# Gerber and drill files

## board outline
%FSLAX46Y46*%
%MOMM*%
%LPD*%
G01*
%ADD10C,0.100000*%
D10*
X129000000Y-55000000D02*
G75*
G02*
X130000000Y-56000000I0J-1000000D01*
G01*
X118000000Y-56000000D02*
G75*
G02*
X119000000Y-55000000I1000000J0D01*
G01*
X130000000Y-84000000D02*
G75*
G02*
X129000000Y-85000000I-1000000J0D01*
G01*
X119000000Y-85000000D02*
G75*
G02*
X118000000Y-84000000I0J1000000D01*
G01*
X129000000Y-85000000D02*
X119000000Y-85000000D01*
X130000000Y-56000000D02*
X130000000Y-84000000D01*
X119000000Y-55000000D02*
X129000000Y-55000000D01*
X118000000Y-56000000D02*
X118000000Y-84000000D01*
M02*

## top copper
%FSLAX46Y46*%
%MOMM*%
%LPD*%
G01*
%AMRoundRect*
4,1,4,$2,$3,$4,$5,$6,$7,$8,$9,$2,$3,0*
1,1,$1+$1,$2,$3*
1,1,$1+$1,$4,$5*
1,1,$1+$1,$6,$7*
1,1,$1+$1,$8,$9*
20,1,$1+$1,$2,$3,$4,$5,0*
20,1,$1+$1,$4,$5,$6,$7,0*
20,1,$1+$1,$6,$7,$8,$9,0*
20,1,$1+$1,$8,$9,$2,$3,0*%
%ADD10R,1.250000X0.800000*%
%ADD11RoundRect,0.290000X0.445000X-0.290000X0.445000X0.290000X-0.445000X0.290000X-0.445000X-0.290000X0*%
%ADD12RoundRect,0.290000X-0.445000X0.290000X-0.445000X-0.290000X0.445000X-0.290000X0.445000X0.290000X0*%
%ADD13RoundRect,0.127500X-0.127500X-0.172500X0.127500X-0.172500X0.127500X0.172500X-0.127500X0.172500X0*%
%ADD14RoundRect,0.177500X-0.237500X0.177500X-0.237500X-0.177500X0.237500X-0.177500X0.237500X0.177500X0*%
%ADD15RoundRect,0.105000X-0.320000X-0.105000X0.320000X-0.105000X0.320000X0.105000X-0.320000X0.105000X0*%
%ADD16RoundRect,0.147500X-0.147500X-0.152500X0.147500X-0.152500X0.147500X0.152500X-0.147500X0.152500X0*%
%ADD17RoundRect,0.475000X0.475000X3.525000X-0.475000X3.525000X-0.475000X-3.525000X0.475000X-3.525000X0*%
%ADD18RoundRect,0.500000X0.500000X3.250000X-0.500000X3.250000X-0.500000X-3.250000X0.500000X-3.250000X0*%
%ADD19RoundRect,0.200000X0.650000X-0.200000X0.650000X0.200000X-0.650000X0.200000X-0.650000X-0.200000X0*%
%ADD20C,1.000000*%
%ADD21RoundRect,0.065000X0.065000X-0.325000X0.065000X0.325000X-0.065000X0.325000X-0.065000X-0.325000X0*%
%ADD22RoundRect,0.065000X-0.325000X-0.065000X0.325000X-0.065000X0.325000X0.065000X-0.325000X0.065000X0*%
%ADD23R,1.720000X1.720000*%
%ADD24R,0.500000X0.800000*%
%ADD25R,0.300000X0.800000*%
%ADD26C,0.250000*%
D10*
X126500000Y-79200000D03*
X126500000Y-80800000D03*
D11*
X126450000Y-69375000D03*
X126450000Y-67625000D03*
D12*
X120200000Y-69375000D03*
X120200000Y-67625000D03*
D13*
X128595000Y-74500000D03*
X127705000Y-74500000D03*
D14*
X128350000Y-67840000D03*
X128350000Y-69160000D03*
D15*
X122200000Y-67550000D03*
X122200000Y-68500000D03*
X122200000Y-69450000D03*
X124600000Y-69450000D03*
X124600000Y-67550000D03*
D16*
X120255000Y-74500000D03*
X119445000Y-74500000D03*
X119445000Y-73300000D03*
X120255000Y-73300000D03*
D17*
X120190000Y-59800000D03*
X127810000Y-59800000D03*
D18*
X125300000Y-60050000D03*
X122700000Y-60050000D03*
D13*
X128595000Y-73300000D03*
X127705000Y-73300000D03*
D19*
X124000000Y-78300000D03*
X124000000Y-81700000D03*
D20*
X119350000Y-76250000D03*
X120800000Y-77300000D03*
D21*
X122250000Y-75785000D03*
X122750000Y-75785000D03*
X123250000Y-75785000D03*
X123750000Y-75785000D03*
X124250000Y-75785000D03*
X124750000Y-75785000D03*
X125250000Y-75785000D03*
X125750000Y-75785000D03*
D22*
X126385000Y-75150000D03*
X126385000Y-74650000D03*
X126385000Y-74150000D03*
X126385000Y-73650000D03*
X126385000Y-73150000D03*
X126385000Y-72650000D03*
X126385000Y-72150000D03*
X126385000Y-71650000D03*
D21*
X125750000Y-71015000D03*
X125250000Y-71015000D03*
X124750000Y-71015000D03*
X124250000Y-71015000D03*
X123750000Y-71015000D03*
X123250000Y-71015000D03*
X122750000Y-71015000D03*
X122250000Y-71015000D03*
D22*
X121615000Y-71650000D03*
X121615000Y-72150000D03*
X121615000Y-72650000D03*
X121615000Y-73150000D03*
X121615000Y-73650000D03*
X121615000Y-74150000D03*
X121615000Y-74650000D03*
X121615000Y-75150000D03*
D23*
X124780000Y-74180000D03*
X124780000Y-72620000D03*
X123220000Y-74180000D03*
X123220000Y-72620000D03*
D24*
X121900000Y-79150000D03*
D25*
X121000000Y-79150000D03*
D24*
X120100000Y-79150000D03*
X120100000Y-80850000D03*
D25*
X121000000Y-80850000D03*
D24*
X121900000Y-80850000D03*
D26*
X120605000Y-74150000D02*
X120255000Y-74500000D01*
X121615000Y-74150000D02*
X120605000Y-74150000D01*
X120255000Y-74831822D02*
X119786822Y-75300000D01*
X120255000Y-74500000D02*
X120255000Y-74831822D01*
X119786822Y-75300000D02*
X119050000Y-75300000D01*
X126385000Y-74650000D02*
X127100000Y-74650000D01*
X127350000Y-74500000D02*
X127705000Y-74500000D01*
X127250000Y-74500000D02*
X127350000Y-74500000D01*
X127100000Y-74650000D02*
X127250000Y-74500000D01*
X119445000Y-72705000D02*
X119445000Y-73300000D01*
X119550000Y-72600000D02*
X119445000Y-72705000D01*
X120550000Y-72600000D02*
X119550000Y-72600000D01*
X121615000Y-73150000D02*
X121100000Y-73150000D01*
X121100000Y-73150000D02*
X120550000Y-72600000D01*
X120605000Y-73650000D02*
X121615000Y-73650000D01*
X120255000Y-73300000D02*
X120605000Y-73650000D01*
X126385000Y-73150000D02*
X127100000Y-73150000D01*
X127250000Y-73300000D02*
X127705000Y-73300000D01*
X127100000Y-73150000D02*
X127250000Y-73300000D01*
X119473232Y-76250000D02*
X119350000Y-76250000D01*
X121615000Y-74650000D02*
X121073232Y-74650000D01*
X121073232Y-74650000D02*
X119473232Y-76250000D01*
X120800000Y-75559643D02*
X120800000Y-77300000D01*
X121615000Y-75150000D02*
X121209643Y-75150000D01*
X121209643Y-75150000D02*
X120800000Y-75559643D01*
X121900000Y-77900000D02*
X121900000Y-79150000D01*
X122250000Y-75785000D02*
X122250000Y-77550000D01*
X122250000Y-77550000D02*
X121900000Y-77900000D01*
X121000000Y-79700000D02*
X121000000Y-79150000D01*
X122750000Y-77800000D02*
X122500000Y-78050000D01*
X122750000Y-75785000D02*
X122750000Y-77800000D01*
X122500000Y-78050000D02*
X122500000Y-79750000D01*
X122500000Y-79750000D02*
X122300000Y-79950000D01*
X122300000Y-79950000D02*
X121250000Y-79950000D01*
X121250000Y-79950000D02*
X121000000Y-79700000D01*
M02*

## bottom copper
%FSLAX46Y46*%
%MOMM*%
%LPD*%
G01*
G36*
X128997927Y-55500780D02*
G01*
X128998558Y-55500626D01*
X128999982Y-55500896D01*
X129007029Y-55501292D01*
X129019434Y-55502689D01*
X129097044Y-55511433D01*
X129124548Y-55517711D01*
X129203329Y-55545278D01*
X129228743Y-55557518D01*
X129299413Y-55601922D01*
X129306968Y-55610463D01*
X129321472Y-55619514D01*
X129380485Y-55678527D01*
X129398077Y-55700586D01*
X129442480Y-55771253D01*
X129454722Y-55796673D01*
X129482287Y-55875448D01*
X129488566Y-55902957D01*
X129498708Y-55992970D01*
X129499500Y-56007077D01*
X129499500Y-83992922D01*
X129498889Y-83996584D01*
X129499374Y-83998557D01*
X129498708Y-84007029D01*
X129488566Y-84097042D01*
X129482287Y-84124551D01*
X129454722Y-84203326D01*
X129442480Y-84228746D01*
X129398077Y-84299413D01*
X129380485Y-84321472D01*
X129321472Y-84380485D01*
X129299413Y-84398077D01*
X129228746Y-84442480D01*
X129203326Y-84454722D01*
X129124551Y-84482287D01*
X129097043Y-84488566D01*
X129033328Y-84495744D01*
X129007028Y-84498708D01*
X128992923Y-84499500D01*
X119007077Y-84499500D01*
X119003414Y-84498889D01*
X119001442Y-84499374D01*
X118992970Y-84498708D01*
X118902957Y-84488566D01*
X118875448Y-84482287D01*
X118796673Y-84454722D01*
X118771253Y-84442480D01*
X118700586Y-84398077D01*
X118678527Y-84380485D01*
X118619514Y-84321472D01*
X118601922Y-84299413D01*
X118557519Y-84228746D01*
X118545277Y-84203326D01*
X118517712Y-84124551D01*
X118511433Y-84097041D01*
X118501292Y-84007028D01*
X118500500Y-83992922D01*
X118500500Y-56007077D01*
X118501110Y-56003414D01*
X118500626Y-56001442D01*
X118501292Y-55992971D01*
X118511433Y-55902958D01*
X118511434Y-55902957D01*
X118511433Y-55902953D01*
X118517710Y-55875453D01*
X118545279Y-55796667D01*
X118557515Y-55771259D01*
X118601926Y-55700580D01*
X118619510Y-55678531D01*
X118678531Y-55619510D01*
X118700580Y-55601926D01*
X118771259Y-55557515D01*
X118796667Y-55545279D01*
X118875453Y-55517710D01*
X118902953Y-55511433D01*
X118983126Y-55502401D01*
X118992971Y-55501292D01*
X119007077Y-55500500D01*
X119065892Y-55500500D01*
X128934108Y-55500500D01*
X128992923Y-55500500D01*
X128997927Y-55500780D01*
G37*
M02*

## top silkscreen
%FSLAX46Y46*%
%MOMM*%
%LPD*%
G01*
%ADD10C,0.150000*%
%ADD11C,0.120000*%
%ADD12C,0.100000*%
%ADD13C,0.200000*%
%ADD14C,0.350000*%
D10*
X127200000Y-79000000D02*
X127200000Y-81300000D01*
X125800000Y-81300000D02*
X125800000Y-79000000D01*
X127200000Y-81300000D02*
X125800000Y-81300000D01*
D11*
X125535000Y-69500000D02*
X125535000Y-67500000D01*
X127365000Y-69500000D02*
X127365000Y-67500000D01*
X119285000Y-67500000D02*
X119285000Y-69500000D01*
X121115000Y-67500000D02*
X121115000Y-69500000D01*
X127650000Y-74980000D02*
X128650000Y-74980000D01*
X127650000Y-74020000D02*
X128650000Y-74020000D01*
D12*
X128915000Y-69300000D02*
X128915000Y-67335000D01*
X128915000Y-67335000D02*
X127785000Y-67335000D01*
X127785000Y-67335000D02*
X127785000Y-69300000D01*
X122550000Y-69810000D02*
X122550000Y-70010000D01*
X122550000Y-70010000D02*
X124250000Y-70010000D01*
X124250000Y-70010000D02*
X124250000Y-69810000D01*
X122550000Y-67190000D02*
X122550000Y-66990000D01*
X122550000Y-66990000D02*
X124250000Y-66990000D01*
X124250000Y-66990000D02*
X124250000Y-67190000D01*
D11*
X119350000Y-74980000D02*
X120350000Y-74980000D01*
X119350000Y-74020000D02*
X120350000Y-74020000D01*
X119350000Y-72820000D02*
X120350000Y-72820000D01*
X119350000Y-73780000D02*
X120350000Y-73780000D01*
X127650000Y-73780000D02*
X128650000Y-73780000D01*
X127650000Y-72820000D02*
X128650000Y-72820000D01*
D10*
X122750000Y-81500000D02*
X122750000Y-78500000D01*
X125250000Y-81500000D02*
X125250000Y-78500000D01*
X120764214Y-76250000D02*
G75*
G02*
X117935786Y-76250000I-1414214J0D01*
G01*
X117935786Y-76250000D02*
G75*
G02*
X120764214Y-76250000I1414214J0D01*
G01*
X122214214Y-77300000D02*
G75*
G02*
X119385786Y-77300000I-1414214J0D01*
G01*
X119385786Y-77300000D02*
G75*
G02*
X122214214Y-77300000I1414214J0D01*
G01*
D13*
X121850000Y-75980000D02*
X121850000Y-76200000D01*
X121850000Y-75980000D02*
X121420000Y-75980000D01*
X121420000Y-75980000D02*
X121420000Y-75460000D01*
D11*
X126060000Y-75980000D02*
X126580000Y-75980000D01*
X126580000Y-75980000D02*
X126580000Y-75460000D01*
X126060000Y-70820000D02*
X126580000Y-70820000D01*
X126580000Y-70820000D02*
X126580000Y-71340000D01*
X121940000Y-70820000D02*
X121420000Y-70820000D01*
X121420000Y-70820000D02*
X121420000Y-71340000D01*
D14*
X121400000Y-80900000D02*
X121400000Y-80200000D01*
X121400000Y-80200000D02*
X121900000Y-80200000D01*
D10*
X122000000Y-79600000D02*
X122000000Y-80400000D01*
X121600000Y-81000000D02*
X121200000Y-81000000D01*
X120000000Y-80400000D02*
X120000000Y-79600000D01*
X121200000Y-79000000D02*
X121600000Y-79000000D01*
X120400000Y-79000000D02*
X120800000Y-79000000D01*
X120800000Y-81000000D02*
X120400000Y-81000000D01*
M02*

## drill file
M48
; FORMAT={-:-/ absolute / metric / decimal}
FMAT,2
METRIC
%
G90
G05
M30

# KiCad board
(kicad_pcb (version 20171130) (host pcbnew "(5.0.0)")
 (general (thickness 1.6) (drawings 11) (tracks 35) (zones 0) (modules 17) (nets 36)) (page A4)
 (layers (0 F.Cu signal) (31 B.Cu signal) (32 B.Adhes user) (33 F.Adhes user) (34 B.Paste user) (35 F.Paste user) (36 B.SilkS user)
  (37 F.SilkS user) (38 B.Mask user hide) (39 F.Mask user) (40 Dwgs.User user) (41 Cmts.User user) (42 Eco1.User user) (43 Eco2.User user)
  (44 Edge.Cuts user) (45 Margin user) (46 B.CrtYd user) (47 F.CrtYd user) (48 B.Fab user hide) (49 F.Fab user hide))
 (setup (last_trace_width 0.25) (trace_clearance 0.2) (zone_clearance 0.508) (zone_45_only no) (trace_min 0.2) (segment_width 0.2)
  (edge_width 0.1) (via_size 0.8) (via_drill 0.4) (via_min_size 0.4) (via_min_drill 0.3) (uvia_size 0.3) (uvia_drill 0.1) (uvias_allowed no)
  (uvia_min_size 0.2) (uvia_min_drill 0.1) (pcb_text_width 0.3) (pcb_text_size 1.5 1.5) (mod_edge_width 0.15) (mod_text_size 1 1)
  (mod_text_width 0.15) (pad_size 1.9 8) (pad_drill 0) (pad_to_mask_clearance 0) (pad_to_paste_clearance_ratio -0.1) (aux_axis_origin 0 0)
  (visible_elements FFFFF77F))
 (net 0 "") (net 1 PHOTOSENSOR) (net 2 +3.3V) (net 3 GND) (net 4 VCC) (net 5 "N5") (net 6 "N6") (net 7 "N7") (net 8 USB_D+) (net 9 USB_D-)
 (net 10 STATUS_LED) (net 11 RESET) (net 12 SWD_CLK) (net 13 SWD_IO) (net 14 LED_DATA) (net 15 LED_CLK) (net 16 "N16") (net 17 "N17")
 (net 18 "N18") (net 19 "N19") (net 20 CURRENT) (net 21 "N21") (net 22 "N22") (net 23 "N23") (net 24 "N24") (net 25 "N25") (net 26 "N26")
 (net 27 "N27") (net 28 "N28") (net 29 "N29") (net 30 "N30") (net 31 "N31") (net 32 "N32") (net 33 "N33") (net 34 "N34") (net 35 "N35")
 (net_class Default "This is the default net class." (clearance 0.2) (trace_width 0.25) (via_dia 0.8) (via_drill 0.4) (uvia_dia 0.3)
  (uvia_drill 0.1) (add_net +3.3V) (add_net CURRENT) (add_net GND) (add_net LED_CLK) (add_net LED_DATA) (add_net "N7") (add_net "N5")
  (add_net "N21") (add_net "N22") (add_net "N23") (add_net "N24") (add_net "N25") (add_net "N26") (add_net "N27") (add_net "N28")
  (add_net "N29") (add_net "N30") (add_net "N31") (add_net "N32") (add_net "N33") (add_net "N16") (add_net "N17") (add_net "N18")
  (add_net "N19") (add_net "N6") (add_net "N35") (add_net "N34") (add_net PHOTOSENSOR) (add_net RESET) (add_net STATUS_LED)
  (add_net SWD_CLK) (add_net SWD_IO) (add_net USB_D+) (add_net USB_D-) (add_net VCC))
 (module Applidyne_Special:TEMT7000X (layer F.Cu) (at 126.5 80 270)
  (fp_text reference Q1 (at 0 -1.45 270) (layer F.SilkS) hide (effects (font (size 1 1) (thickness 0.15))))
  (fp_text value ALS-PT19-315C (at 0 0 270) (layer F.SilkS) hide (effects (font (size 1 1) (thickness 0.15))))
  (fp_line (start -1 -0.7) (end 1.3 -0.7) (layer F.SilkS) (width 0.15))
  (fp_line (start 1.3 0.7) (end -1 0.7) (layer F.SilkS) (width 0.15))
  (fp_line (start 1.3 -0.7) (end 1.3 0.7) (layer F.SilkS) (width 0.15))
  (pad E smd rect (at -0.8 0 270) (size 0.8 1.25) (layers F.Cu F.Paste F.Mask) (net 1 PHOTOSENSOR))
  (pad C smd rect (at 0.8 0 270) (size 0.8 1.25) (layers F.Cu F.Paste F.Mask) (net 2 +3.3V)))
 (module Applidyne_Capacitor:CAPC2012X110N (layer F.Cu) (at 126.45 68.5 270) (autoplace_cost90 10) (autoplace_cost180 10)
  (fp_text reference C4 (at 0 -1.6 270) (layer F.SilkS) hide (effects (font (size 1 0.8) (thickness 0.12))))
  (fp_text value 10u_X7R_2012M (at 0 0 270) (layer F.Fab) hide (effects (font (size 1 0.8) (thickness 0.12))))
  (fp_line (start 1 0.915) (end -1 0.915) (layer F.SilkS) (width 0.12))
  (fp_line (start 1 -0.915) (end -1 -0.915) (layer F.SilkS) (width 0.12))
  (pad 2 smd roundrect (at 0.875 0 90) (size 1.16 1.47) (layers F.Cu F.Paste F.Mask) (roundrect_rratio 0.25) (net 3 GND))
  (pad 1 smd roundrect (at -0.875 0 90) (size 1.16 1.47) (layers F.Cu F.Paste F.Mask) (roundrect_rratio 0.25) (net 2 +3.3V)))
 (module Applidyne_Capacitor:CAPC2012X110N (layer F.Cu) (at 120.2 68.5 90) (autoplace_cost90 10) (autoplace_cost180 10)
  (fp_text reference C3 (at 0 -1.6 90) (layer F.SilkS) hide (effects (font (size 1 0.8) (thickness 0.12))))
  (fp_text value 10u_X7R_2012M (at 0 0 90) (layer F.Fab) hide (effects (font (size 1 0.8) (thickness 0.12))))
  (fp_line (start 1 -0.915) (end -1 -0.915) (layer F.SilkS) (width 0.12))
  (fp_line (start 1 0.915) (end -1 0.915) (layer F.SilkS) (width 0.12))
  (pad 1 smd roundrect (at -0.875 0 270) (size 1.16 1.47) (layers F.Cu F.Paste F.Mask) (roundrect_rratio 0.25) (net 3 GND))
  (pad 2 smd roundrect (at 0.875 0 270) (size 1.16 1.47) (layers F.Cu F.Paste F.Mask) (roundrect_rratio 0.25) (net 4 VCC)))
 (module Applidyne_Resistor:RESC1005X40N (layer F.Cu) (at 128.15 74.5 180) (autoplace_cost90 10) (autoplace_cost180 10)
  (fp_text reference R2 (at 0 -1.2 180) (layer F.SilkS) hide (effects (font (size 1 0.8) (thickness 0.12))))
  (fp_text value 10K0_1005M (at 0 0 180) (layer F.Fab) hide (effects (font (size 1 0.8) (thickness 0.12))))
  (fp_line (start 0.5 -0.48) (end -0.5 -0.48) (layer F.SilkS) (width 0.12))
  (fp_line (start 0.5 0.48) (end -0.5 0.48) (layer F.SilkS) (width 0.12))
  (pad 1 smd roundrect (at -0.445 0) (size 0.51 0.6) (layers F.Cu F.Paste F.Mask) (roundrect_rratio 0.25) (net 1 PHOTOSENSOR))
  (pad 2 smd roundrect (at 0.445 0) (size 0.51 0.6) (layers F.Cu F.Paste F.Mask) (roundrect_rratio 0.25) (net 3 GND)))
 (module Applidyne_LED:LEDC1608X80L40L (layer F.Cu) (at 128.35 68.5 270)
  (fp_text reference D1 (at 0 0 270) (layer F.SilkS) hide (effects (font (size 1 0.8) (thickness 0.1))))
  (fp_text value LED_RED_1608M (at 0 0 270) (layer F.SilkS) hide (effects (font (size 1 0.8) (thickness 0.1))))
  (fp_line (start 0.8 -0.565) (end -1.165 -0.565) (layer F.SilkS) (width 0.1))
  (fp_line (start -1.165 -0.565) (end -1.165 0.565) (layer F.SilkS) (width 0.1))
  (fp_line (start -1.165 0.565) (end 0.8 0.565) (layer F.SilkS) (width 0.1))
  (pad C smd roundrect (at -0.66 0 270) (size 0.71 0.83) (layers F.Cu F.Paste F.Mask) (roundrect_rratio 0.25) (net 3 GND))
  (pad A smd roundrect (at 0.66 0 270) (size 0.71 0.83) (layers F.Cu F.Paste F.Mask) (roundrect_rratio 0.25) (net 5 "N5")))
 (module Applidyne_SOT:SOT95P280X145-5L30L (layer F.Cu) (at 123.4 68.5 270)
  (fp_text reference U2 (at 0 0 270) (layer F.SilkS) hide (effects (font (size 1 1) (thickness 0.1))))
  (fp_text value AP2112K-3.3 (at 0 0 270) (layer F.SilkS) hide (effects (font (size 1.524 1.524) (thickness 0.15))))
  (fp_line (start 1.31 0.85) (end 1.51 0.85) (layer F.SilkS) (width 0.1))
  (fp_line (start 1.51 0.85) (end 1.51 -0.85) (layer F.SilkS) (width 0.1))
  (fp_line (start 1.51 -0.85) (end 1.31 -0.85) (layer F.SilkS) (width 0.1))
  (fp_line (start -1.31 0.85) (end -1.51 0.85) (layer F.SilkS) (width 0.1))
  (fp_line (start -1.51 0.85) (end -1.51 -0.85) (layer F.SilkS) (width 0.1))
  (fp_line (start -1.51 -0.85) (end -1.31 -0.85) (layer F.SilkS) (width 0.1))
  (pad 1 smd roundrect (at -0.95 1.2) (size 0.85 0.42) (layers F.Cu F.Paste F.Mask) (roundrect_rratio 0.25) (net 4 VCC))
  (pad 2 smd roundrect (at 0 1.2) (size 0.85 0.42) (layers F.Cu F.Paste F.Mask) (roundrect_rratio 0.25) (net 3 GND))
  (pad 3 smd roundrect (at 0.95 1.2) (size 0.85 0.42) (layers F.Cu F.Paste F.Mask) (roundrect_rratio 0.25) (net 4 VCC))
  (pad 4 smd roundrect (at 0.95 -1.2) (size 0.85 0.42) (layers F.Cu F.Paste F.Mask) (roundrect_rratio 0.25) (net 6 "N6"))
  (pad 5 smd roundrect (at -0.95 -1.2) (size 0.85 0.42) (layers F.Cu F.Paste F.Mask) (roundrect_rratio 0.25) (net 2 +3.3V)))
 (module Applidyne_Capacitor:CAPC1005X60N (layer F.Cu) (at 119.85 74.5 180) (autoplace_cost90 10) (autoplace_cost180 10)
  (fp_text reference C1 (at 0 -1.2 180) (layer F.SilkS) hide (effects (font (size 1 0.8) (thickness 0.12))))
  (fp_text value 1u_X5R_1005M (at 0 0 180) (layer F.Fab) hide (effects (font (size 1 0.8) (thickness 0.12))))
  (fp_line (start 0.5 -0.48) (end -0.5 -0.48) (layer F.SilkS) (width 0.12))
  (fp_line (start 0.5 0.48) (end -0.5 0.48) (layer F.SilkS) (width 0.12))
  (pad 1 smd roundrect (at -0.405 0) (size 0.59 0.6) (layers F.Cu F.Paste F.Mask) (roundrect_rratio 0.25) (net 2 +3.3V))
  (pad 2 smd roundrect (at 0.405 0) (size 0.59 0.6) (layers F.Cu F.Paste F.Mask) (roundrect_rratio 0.25) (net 3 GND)))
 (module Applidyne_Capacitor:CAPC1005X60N (layer F.Cu) (at 119.85 73.3 180) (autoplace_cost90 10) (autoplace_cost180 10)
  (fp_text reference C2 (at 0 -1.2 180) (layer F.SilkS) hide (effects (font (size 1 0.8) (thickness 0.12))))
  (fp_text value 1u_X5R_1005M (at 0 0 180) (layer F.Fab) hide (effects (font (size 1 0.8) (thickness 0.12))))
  (fp_line (start 0.5 0.48) (end -0.5 0.48) (layer F.SilkS) (width 0.12))
  (fp_line (start 0.5 -0.48) (end -0.5 -0.48) (layer F.SilkS) (width 0.12))
  (pad 2 smd roundrect (at 0.405 0) (size 0.59 0.6) (layers F.Cu F.Paste F.Mask) (roundrect_rratio 0.25) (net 3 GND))
  (pad 1 smd roundrect (at -0.405 0) (size 0.59 0.6) (layers F.Cu F.Paste F.Mask) (roundrect_rratio 0.25) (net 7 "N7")))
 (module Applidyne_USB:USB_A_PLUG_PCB (layer F.Cu) (at 124 54.9 180)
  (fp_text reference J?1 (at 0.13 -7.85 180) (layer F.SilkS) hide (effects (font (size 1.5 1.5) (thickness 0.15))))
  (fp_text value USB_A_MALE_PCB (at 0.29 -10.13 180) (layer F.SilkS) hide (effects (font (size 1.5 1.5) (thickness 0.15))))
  (pad 1 connect roundrect (at 3.81 -4.9 180) (size 1.9 8) (layers F.Cu F.Mask) (roundrect_rratio 0.25) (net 4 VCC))
  (pad 4 connect roundrect (at -3.81 -4.9 180) (size 1.9 8) (layers F.Cu F.Mask) (roundrect_rratio 0.25) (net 3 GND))
  (pad 3 connect roundrect (at -1.3 -5.15 180) (size 2 7.5) (layers F.Cu F.Mask) (roundrect_rratio 0.25) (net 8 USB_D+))
  (pad 2 connect roundrect (at 1.3 -5.15 180) (size 2 7.5) (layers F.Cu F.Mask) (roundrect_rratio 0.25) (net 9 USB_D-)))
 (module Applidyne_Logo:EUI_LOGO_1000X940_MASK (layer B.Cu) (at 124 72.95 180)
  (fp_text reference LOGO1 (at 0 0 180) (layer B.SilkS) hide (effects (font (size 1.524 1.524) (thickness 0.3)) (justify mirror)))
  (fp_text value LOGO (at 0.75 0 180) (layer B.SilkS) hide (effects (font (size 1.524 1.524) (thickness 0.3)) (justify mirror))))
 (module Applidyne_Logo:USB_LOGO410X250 (layer B.Cu) (at 124 59.8 90)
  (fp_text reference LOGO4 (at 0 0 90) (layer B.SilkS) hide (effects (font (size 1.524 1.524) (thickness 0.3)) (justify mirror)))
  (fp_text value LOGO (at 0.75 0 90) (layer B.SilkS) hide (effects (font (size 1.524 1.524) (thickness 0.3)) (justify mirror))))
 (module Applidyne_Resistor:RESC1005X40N (layer F.Cu) (at 128.15 73.3 180) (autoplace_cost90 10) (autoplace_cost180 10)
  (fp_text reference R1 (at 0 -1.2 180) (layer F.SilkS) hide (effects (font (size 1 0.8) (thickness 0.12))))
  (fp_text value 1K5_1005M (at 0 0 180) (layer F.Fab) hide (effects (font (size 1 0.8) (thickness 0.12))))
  (fp_line (start 0.5 -0.48) (end -0.5 -0.48) (layer F.SilkS) (width 0.12))
  (fp_line (start 0.5 0.48) (end -0.5 0.48) (layer F.SilkS) (width 0.12))
  (pad 1 smd roundrect (at -0.445 0) (size 0.51 0.6) (layers F.Cu F.Paste F.Mask) (roundrect_rratio 0.25) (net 5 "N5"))
  (pad 2 smd roundrect (at 0.445 0) (size 0.51 0.6) (layers F.Cu F.Paste F.Mask) (roundrect_rratio 0.25) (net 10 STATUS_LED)))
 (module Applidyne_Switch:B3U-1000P (layer F.Cu) (at 124 80 90)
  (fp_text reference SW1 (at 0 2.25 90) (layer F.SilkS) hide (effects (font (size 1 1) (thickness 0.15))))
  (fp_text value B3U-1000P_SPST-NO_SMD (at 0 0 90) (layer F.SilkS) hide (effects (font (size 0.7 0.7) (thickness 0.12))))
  (fp_line (start -1.5 -1.25) (end 1.5 -1.25) (layer F.SilkS) (width 0.15))
  (fp_line (start -1.5 1.25) (end 1.5 1.25) (layer F.SilkS) (width 0.15))
  (pad 1 smd roundrect (at 1.7 0 90) (size 0.8 1.7) (layers F.Cu F.Paste F.Mask) (roundrect_rratio 0.25) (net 3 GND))
  (pad 2 smd roundrect (at -1.7 0 90) (size 0.8 1.7) (layers F.Cu F.Paste F.Mask) (roundrect_rratio 0.25) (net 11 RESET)))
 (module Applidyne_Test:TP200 (layer F.Cu) (at 119.35 76.25)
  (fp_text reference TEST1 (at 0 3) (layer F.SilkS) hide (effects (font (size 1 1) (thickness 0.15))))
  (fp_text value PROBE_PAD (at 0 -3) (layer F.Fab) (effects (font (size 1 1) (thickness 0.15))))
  (fp_circle (center 0 0) (end 1 1) (layer F.SilkS) (width 0.15))
  (pad 1 smd circle (at 0 0) (size 1 1) (layers F.Cu F.Mask) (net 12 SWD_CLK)))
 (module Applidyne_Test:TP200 (layer F.Cu) (at 120.8 77.3)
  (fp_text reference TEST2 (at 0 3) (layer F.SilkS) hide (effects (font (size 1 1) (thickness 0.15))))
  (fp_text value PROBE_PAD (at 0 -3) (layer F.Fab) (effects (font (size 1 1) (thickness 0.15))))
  (fp_circle (center 0 0) (end 1 1) (layer F.SilkS) (width 0.15))
  (pad 1 smd circle (at 0 0) (size 1 1) (layers F.Cu F.Mask) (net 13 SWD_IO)))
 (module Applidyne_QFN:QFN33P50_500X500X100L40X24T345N (layer F.Cu) (at 124 73.4)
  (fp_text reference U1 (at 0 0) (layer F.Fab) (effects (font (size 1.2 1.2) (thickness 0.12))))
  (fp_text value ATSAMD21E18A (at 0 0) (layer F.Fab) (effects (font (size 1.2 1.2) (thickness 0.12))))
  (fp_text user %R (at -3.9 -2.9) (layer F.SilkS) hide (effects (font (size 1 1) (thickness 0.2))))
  (fp_line (start -2.15 2.58) (end -2.15 2.8) (layer F.SilkS) (width 0.2))
  (fp_line (start -2.15 2.58) (end -2.58 2.58) (layer F.SilkS) (width 0.2))
  (fp_line (start -2.58 2.58) (end -2.58 2.06) (layer F.SilkS) (width 0.2))
  (fp_line (start 2.06 2.58) (end 2.58 2.58) (layer F.SilkS) (width 0.12))
  (fp_line (start 2.58 2.58) (end 2.58 2.06) (layer F.SilkS) (width 0.12))
  (fp_line (start 2.06 -2.58) (end 2.58 -2.58) (layer F.SilkS) (width 0.12))
  (fp_line (start 2.58 -2.58) (end 2.58 -2.06) (layer F.SilkS) (width 0.12))
  (fp_line (start -2.06 -2.58) (end -2.58 -2.58) (layer F.SilkS) (width 0.12))
  (fp_line (start -2.58 -2.58) (end -2.58 -2.06) (layer F.SilkS) (width 0.12))
  (pad 1 smd roundrect (at -1.75 2.385 90) (size 0.78 0.26) (layers F.Cu F.Paste F.Mask) (roundrect_rratio 0.25) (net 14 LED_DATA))
  (pad 2 smd roundrect (at -1.25 2.385 90) (size 0.78 0.26) (layers F.Cu F.Paste F.Mask) (roundrect_rratio 0.25) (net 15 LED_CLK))
  (pad 3 smd roundrect (at -0.75 2.385 90) (size 0.78 0.26) (layers F.Cu F.Paste F.Mask) (roundrect_rratio 0.25) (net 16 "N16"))
  (pad 4 smd roundrect (at -0.25 2.385 90) (size 0.78 0.26) (layers F.Cu F.Paste F.Mask) (roundrect_rratio 0.25) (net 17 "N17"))
  (pad 5 smd roundrect (at 0.25 2.385 90) (size 0.78 0.26) (layers F.Cu F.Paste F.Mask) (roundrect_rratio 0.25) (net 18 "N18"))
  (pad 6 smd roundrect (at 0.75 2.385 90) (size 0.78 0.26) (layers F.Cu F.Paste F.Mask) (roundrect_rratio 0.25) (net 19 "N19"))
  (pad 7 smd roundrect (at 1.25 2.385 90) (size 0.78 0.26) (layers F.Cu F.Paste F.Mask) (roundrect_rratio 0.25) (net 1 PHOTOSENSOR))
  (pad 8 smd roundrect (at 1.75 2.385 90) (size 0.78 0.26) (layers F.Cu F.Paste F.Mask) (roundrect_rratio 0.25) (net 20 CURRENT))
  (pad 9 smd roundrect (at 2.385 1.75) (size 0.78 0.26) (layers F.Cu F.Paste F.Mask) (roundrect_rratio 0.25) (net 2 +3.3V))
  (pad 10 smd roundrect (at 2.385 1.25) (size 0.78 0.26) (layers F.Cu F.Paste F.Mask) (roundrect_rratio 0.25) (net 3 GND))
  (pad 11 smd roundrect (at 2.385 0.75) (size 0.78 0.26) (layers F.Cu F.Paste F.Mask) (roundrect_rratio 0.25) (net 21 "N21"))
  (pad 12 smd roundrect (at 2.385 0.25) (size 0.78 0.26) (layers F.Cu F.Paste F.Mask) (roundrect_rratio 0.25) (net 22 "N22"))
  (pad 13 smd roundrect (at 2.385 -0.25) (size 0.78 0.26) (layers F.Cu F.Paste F.Mask) (roundrect_rratio 0.25) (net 10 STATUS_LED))
  (pad 14 smd roundrect (at 2.385 -0.75) (size 0.78 0.26) (layers F.Cu F.Paste F.Mask) (roundrect_rratio 0.25) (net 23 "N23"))
  (pad 15 smd roundrect (at 2.385 -1.25) (size 0.78 0.26) (layers F.Cu F.Paste F.Mask) (roundrect_rratio 0.25) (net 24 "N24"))
  (pad 16 smd roundrect (at 2.385 -1.75) (size 0.78 0.26) (layers F.Cu F.Paste F.Mask) (roundrect_rratio 0.25) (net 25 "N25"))
  (pad 17 smd roundrect (at 1.75 -2.385 90) (size 0.78 0.26) (layers F.Cu F.Paste F.Mask) (roundrect_rratio 0.25) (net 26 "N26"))
  (pad 18 smd roundrect (at 1.25 -2.385 90) (size 0.78 0.26) (layers F.Cu F.Paste F.Mask) (roundrect_rratio 0.25) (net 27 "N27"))
  (pad 19 smd roundrect (at 0.75 -2.385 90) (size 0.78 0.26) (layers F.Cu F.Paste F.Mask) (roundrect_rratio 0.25) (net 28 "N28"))
  (pad 20 smd roundrect (at 0.25 -2.385 90) (size 0.78 0.26) (layers F.Cu F.Paste F.Mask) (roundrect_rratio 0.25) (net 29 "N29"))
  (pad 21 smd roundrect (at -0.25 -2.385 90) (size 0.78 0.26) (layers F.Cu F.Paste F.Mask) (roundrect_rratio 0.25) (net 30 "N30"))
  (pad 22 smd roundrect (at -0.75 -2.385 90) (size 0.78 0.26) (layers F.Cu F.Paste F.Mask) (roundrect_rratio 0.25) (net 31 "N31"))
  (pad 23 smd roundrect (at -1.25 -2.385 90) (size 0.78 0.26) (layers F.Cu F.Paste F.Mask) (roundrect_rratio 0.25) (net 9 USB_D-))
  (pad 24 smd roundrect (at -1.75 -2.385 90) (size 0.78 0.26) (layers F.Cu F.Paste F.Mask) (roundrect_rratio 0.25) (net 8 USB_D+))
  (pad 25 smd roundrect (at -2.385 -1.75) (size 0.78 0.26) (layers F.Cu F.Paste F.Mask) (roundrect_rratio 0.25) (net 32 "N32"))
  (pad 26 smd roundrect (at -2.385 -1.25) (size 0.78 0.26) (layers F.Cu F.Paste F.Mask) (roundrect_rratio 0.25) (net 11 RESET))
  (pad 27 smd roundrect (at -2.385 -0.75) (size 0.78 0.26) (layers F.Cu F.Paste F.Mask) (roundrect_rratio 0.25) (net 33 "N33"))
  (pad 28 smd roundrect (at -2.385 -0.25) (size 0.78 0.26) (layers F.Cu F.Paste F.Mask) (roundrect_rratio 0.25) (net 3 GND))
  (pad 29 smd roundrect (at -2.385 0.25) (size 0.78 0.26) (layers F.Cu F.Paste F.Mask) (roundrect_rratio 0.25) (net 7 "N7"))
  (pad 30 smd roundrect (at -2.385 0.75) (size 0.78 0.26) (layers F.Cu F.Paste F.Mask) (roundrect_rratio 0.25) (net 2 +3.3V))
  (pad 31 smd roundrect (at -2.385 1.25) (size 0.78 0.26) (layers F.Cu F.Paste F.Mask) (roundrect_rratio 0.25) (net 12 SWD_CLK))
  (pad 32 smd roundrect (at -2.385 1.75) (size 0.78 0.26) (layers F.Cu F.Paste F.Mask) (roundrect_rratio 0.25) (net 13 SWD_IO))
  (pad 33 smd rect (at 0.78 0.78) (size 1.72 1.72) (layers F.Cu F.Paste F.Mask) (solder_paste_margin_ratio -0.29))
  (pad 33 smd rect (at 0.78 -0.78) (size 1.72 1.72) (layers F.Cu F.Paste F.Mask) (solder_paste_margin_ratio -0.29))
  (pad 33 smd rect (at -0.78 0.78) (size 1.72 1.72) (layers F.Cu F.Paste F.Mask) (solder_paste_margin_ratio -0.29))
  (pad 33 smd rect (at -0.78 -0.78) (size 1.72 1.72) (layers F.Cu F.Paste F.Mask) (solder_paste_margin_ratio -0.29))
  (pad "" smd rect (at 0.78 0.78 90) (size 1.22 1.22) (layers F.Paste))
  (pad "" smd rect (at 0.78 -0.78 90) (size 1.22 1.22) (layers F.Paste))
  (pad "" smd rect (at -0.78 0.78 90) (size 1.22 1.22) (layers F.Paste))
  (pad "" smd rect (at -0.78 -0.78 90) (size 1.22 1.22) (layers F.Paste)))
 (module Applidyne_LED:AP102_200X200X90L (layer F.Cu) (at 121 80 270)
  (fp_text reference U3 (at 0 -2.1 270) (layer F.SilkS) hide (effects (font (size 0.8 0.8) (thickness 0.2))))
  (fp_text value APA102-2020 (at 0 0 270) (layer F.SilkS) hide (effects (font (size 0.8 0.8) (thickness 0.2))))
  (fp_line (start 0.9 -0.4) (end 0.2 -0.4) (layer F.SilkS) (width 0.35))
  (fp_line (start 0.2 -0.4) (end 0.2 -0.9) (layer F.SilkS) (width 0.35))
  (fp_line (start -0.4 -1) (end 0.4 -1) (layer F.SilkS) (width 0.15))
  (fp_line (start 1 -0.6) (end 1 -0.2) (layer F.SilkS) (width 0.15))
  (fp_line (start 0.4 1) (end -0.4 1) (layer F.SilkS) (width 0.15))
  (fp_line (start -1 -0.2) (end -1 -0.6) (layer F.SilkS) (width 0.15))
  (fp_line (start -1 0.6) (end -1 0.2) (layer F.SilkS) (width 0.15))
  (fp_line (start 1 0.2) (end 1 0.6) (layer F.SilkS) (width 0.15))
  (pad 2 smd rect (at -0.85 -0.9 270) (size 0.8 0.5) (layers F.Cu F.Paste F.Mask) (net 14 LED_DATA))
  (pad 3 smd rect (at -0.85 0 270) (size 0.8 0.3) (layers F.Cu F.Paste F.Mask) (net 15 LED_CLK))
  (pad 4 smd rect (at -0.85 0.9 270) (size 0.8 0.5) (layers F.Cu F.Paste F.Mask) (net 3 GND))
  (pad 5 smd rect (at 0.85 0.9 270) (size 0.8 0.5) (layers F.Cu F.Paste F.Mask) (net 2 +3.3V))
  (pad 6 smd rect (at 0.85 0 270) (size 0.8 0.3) (layers F.Cu F.Paste F.Mask) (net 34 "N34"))
  (pad 1 smd rect (at 0.85 -0.9 270) (size 0.8 0.5) (layers F.Cu F.Paste F.Mask) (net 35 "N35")))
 (gr_arc (start 129 56) (end 130 56) (angle -90) (layer Edge.Cuts) (width 0.1))
 (gr_arc (start 119 56) (end 119 55) (angle -90) (layer Edge.Cuts) (width 0.1))
 (gr_arc (start 129 84) (end 129 85) (angle -90) (layer Edge.Cuts) (width 0.1))
 (gr_arc (start 119 84) (end 118 84) (angle -90) (layer Edge.Cuts) (width 0.1))
 (gr_line (start 129 85) (end 119 85) (layer Edge.Cuts) (width 0.1))
 (gr_line (start 130 56) (end 130 84) (layer Edge.Cuts) (width 0.1))
 (gr_line (start 119 55) (end 129 55) (layer Edge.Cuts) (width 0.1))
 (gr_line (start 118 56) (end 118 84) (layer Edge.Cuts) (width 0.1))
 (segment (start 120.605 74.15) (end 120.255 74.5) (width 0.25) (layer F.Cu) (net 2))
 (segment (start 121.615 74.15) (end 120.605 74.15) (width 0.25) (layer F.Cu) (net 2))
 (segment (start 120.255 74.831822) (end 119.786822 75.3) (width 0.25) (layer F.Cu) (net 2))
 (segment (start 120.255 74.5) (end 120.255 74.831822) (width 0.25) (layer F.Cu) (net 2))
 (segment (start 119.786822 75.3) (end 119.05 75.3) (width 0.25) (layer F.Cu) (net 2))
 (segment (start 126.385 74.65) (end 127.1 74.65) (width 0.25) (layer F.Cu) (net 3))
 (segment (start 127.35 74.5) (end 127.705 74.5) (width 0.25) (layer F.Cu) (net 3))
 (segment (start 127.25 74.5) (end 127.35 74.5) (width 0.25) (layer F.Cu) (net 3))
 (segment (start 127.1 74.65) (end 127.25 74.5) (width 0.25) (layer F.Cu) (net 3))
 (segment (start 119.445 72.705) (end 119.445 73.3) (width 0.25) (layer F.Cu) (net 3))
 (segment (start 119.55 72.6) (end 119.445 72.705) (width 0.25) (layer F.Cu) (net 3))
 (segment (start 120.55 72.6) (end 119.55 72.6) (width 0.25) (layer F.Cu) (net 3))
 (segment (start 121.615 73.15) (end 121.1 73.15) (width 0.25) (layer F.Cu) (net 3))
 (segment (start 121.1 73.15) (end 120.55 72.6) (width 0.25) (layer F.Cu) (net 3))
 (segment (start 120.605 73.65) (end 121.615 73.65) (width 0.25) (layer F.Cu) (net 7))
 (segment (start 120.255 73.3) (end 120.605 73.65) (width 0.25) (layer F.Cu) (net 7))
 (segment (start 126.385 73.15) (end 127.1 73.15) (width 0.25) (layer F.Cu) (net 10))
 (segment (start 127.25 73.3) (end 127.705 73.3) (width 0.25) (layer F.Cu) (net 10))
 (segment (start 127.1 73.15) (end 127.25 73.3) (width 0.25) (layer F.Cu) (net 10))
 (segment (start 119.473232 76.25) (end 119.35 76.25) (width 0.25) (layer F.Cu) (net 12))
 (segment (start 121.615 74.65) (end 121.073232 74.65) (width 0.25) (layer F.Cu) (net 12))
 (segment (start 121.073232 74.65) (end 119.473232 76.25) (width 0.25) (layer F.Cu) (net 12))
 (segment (start 120.8 75.559643) (end 120.8 77.3) (width 0.25) (layer F.Cu) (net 13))
 (segment (start 121.615 75.15) (end 121.209643 75.15) (width 0.25) (layer F.Cu) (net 13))
 (segment (start 121.209643 75.15) (end 120.8 75.559643) (width 0.25) (layer F.Cu) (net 13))
 (segment (start 121.9 77.9) (end 121.9 79.15) (width 0.25) (layer F.Cu) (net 14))
 (segment (start 122.25 75.785) (end 122.25 77.55) (width 0.25) (layer F.Cu) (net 14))
 (segment (start 122.25 77.55) (end 121.9 77.9) (width 0.25) (layer F.Cu) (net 14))
 (segment (start 121 79.7) (end 121 79.15) (width 0.25) (layer F.Cu) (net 15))
 (segment (start 122.75 77.8) (end 122.5 78.05) (width 0.25) (layer F.Cu) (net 15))
 (segment (start 122.75 75.785) (end 122.75 77.8) (width 0.25) (layer F.Cu) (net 15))
 (segment (start 122.5 78.05) (end 122.5 79.75) (width 0.25) (layer F.Cu) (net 15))
 (segment (start 122.5 79.75) (end 122.3 79.95) (width 0.25) (layer F.Cu) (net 15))
 (segment (start 122.3 79.95) (end 121.25 79.95) (width 0.25) (layer F.Cu) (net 15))
 (segment (start 121.25 79.95) (end 121 79.7) (width 0.25) (layer F.Cu) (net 15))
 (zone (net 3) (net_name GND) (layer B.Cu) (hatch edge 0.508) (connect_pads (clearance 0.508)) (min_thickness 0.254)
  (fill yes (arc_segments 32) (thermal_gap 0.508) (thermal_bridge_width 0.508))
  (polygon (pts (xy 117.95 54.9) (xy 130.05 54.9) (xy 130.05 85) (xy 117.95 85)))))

